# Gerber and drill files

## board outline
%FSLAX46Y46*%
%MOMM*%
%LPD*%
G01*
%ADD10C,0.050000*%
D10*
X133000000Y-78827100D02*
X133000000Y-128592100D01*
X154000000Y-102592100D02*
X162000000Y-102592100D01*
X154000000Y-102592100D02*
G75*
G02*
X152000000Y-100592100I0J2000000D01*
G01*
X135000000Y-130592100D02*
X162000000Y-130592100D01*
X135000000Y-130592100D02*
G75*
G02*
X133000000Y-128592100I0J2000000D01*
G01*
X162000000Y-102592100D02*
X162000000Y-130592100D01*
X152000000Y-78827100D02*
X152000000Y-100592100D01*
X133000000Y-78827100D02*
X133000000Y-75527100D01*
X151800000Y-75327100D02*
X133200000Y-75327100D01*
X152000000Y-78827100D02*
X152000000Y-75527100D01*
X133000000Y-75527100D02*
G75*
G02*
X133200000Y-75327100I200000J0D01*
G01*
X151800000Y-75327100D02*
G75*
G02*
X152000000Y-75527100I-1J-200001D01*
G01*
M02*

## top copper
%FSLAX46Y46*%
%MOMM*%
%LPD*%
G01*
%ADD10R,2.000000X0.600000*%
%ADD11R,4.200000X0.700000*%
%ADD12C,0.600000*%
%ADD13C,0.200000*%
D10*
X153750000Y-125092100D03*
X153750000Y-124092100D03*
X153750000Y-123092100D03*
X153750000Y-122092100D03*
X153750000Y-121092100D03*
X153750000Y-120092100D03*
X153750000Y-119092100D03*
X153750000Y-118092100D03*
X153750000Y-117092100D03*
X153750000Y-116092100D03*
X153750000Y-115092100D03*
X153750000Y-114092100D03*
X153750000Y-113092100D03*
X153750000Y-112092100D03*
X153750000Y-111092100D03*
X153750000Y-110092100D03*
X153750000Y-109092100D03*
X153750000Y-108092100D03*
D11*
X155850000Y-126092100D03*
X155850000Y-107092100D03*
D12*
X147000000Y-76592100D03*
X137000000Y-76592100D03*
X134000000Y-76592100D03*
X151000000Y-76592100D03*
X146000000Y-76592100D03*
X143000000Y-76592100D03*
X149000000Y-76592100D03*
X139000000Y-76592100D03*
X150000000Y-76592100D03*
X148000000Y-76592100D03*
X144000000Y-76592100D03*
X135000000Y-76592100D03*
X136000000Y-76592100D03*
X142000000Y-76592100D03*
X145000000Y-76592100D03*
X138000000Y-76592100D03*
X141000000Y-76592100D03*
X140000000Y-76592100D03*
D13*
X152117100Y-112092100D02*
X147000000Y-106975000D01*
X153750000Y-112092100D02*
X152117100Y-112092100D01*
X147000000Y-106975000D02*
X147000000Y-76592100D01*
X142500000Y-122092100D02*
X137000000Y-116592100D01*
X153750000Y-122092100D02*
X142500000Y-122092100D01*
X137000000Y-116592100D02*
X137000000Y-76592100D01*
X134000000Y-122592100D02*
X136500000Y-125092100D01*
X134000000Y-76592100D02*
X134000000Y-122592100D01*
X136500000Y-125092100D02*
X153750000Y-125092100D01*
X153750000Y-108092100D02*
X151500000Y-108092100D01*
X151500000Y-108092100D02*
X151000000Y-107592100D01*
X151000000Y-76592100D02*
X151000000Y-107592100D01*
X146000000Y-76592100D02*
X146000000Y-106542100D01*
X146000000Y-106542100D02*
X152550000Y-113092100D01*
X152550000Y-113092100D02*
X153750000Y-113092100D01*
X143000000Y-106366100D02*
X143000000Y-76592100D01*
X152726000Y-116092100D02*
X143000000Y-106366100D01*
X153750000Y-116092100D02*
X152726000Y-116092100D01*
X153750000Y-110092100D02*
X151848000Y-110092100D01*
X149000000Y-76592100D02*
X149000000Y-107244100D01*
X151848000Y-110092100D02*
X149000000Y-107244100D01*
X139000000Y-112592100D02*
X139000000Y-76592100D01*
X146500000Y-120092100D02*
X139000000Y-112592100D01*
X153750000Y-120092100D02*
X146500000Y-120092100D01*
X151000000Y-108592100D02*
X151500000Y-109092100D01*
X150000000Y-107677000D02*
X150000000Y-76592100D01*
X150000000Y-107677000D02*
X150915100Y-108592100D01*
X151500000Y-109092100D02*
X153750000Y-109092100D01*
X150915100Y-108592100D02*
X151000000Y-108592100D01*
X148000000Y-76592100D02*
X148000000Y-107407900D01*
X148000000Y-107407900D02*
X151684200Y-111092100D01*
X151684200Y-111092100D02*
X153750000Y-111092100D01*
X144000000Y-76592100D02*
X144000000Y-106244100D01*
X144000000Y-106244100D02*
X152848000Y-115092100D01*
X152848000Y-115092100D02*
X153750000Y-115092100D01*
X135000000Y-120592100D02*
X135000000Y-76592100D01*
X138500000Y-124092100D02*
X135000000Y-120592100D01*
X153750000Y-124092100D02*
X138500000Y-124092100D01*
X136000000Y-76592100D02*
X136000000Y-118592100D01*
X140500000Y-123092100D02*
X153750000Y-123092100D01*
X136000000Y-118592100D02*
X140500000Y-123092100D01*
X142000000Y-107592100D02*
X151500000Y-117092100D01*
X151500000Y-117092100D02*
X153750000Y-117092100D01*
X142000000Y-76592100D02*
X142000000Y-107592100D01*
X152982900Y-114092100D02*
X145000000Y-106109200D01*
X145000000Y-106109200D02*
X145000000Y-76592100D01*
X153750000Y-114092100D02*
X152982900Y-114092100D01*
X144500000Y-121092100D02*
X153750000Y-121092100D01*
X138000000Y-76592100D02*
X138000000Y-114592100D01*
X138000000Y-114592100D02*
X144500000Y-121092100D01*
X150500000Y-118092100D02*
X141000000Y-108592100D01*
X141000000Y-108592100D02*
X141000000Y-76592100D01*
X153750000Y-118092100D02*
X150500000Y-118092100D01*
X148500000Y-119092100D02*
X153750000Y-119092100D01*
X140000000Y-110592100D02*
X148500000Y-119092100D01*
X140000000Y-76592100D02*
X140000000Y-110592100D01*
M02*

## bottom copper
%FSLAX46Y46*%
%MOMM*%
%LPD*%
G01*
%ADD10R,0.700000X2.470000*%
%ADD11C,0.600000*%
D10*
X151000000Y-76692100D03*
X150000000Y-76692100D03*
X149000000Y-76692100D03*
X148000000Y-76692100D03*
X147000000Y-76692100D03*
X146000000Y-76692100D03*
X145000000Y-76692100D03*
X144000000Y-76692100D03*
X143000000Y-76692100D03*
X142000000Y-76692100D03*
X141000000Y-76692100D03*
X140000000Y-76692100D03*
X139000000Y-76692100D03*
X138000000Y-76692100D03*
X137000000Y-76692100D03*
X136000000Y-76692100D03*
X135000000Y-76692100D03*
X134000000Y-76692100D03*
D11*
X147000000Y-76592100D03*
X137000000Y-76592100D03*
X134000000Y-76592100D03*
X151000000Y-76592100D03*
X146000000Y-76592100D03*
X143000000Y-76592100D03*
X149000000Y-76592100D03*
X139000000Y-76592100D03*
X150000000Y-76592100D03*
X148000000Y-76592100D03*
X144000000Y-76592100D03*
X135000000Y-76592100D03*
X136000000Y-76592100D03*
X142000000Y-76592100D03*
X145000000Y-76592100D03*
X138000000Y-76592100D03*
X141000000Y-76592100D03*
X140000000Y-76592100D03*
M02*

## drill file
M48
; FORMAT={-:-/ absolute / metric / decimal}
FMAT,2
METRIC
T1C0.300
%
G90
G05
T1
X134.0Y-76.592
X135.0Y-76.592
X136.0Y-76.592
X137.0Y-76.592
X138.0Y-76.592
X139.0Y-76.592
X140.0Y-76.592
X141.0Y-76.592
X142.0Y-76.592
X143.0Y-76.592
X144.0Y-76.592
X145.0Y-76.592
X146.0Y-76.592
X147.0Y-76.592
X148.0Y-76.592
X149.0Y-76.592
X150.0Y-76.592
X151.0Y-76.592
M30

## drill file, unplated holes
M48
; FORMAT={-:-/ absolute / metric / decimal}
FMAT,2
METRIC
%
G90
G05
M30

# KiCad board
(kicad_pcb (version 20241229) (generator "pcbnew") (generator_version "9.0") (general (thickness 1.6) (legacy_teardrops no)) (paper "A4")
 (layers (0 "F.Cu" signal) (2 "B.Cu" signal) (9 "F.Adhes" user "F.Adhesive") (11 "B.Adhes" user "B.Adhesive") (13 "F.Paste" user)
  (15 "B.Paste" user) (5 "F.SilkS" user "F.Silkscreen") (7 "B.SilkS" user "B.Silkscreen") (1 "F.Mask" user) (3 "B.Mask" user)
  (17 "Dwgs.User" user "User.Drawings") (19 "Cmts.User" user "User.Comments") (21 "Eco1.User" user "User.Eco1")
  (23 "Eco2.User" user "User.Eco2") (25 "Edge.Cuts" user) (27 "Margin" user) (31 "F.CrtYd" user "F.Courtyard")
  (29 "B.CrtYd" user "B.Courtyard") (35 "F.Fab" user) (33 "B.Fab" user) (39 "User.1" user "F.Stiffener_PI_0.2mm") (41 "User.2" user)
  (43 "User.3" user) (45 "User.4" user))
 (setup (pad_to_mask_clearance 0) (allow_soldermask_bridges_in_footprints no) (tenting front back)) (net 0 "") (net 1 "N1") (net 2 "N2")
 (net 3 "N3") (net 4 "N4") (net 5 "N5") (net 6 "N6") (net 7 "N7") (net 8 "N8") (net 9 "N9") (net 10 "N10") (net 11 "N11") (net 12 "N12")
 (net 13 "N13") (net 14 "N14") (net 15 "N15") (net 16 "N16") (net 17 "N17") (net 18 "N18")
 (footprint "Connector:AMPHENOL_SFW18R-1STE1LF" (layer "F.Cu") (at 157 116.5921 90)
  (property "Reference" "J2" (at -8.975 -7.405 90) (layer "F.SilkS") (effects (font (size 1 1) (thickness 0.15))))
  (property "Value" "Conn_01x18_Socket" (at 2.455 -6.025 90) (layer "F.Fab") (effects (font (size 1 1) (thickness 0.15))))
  (pad "1" smd rect (at -8.5 -3.25 90) (size 0.6 2) (layers "F.Cu" "F.Mask" "F.Paste") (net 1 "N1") (solder_mask_margin 0.102))
  (pad "2" smd rect (at -7.5 -3.25 90) (size 0.6 2) (layers "F.Cu" "F.Mask" "F.Paste") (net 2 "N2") (solder_mask_margin 0.102))
  (pad "3" smd rect (at -6.5 -3.25 90) (size 0.6 2) (layers "F.Cu" "F.Mask" "F.Paste") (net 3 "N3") (solder_mask_margin 0.102))
  (pad "4" smd rect (at -5.5 -3.25 90) (size 0.6 2) (layers "F.Cu" "F.Mask" "F.Paste") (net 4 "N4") (solder_mask_margin 0.102))
  (pad "5" smd rect (at -4.5 -3.25 90) (size 0.6 2) (layers "F.Cu" "F.Mask" "F.Paste") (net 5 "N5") (solder_mask_margin 0.102))
  (pad "6" smd rect (at -3.5 -3.25 90) (size 0.6 2) (layers "F.Cu" "F.Mask" "F.Paste") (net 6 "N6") (solder_mask_margin 0.102))
  (pad "7" smd rect (at -2.5 -3.25 90) (size 0.6 2) (layers "F.Cu" "F.Mask" "F.Paste") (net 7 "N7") (solder_mask_margin 0.102))
  (pad "8" smd rect (at -1.5 -3.25 90) (size 0.6 2) (layers "F.Cu" "F.Mask" "F.Paste") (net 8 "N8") (solder_mask_margin 0.102))
  (pad "9" smd rect (at -0.5 -3.25 90) (size 0.6 2) (layers "F.Cu" "F.Mask" "F.Paste") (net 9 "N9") (solder_mask_margin 0.102))
  (pad "10" smd rect (at 0.5 -3.25 90) (size 0.6 2) (layers "F.Cu" "F.Mask" "F.Paste") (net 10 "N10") (solder_mask_margin 0.102))
  (pad "11" smd rect (at 1.5 -3.25 90) (size 0.6 2) (layers "F.Cu" "F.Mask" "F.Paste") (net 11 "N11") (solder_mask_margin 0.102))
  (pad "12" smd rect (at 2.5 -3.25 90) (size 0.6 2) (layers "F.Cu" "F.Mask" "F.Paste") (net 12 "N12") (solder_mask_margin 0.102))
  (pad "13" smd rect (at 3.5 -3.25 90) (size 0.6 2) (layers "F.Cu" "F.Mask" "F.Paste") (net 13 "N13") (solder_mask_margin 0.102))
  (pad "14" smd rect (at 4.5 -3.25 90) (size 0.6 2) (layers "F.Cu" "F.Mask" "F.Paste") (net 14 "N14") (solder_mask_margin 0.102))
  (pad "15" smd rect (at 5.5 -3.25 90) (size 0.6 2) (layers "F.Cu" "F.Mask" "F.Paste") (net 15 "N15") (solder_mask_margin 0.102))
  (pad "16" smd rect (at 6.5 -3.25 90) (size 0.6 2) (layers "F.Cu" "F.Mask" "F.Paste") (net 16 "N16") (solder_mask_margin 0.102))
  (pad "17" smd rect (at 7.5 -3.25 90) (size 0.6 2) (layers "F.Cu" "F.Mask" "F.Paste") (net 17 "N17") (solder_mask_margin 0.102))
  (pad "18" smd rect (at 8.5 -3.25 90) (size 0.6 2) (layers "F.Cu" "F.Mask" "F.Paste") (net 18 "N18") (solder_mask_margin 0.102))
  (pad "S1" smd rect (at -9.5 -1.15 90) (size 0.7 4.2) (layers "F.Cu" "F.Mask" "F.Paste") (solder_mask_margin 0.102))
  (pad "S2" smd rect (at 9.5 -1.15 90) (size 0.7 4.2) (layers "F.Cu" "F.Mask" "F.Paste") (solder_mask_margin 0.102)))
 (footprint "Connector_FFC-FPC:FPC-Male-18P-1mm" (layer "B.Cu") (at 142.91 76.6321 180)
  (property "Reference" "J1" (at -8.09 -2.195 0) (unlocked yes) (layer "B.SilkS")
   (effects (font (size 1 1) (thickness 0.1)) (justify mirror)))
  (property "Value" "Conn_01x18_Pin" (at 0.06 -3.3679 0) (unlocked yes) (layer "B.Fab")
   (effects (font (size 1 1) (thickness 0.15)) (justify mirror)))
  (fp_line (start 9.91 -2.195) (end 9.91 1.105) (stroke (width 0.05) (type default)) (layer "Edge.Cuts"))
  (fp_line (start -8.89 1.305) (end 9.71 1.305) (stroke (width 0.05) (type default)) (layer "Edge.Cuts"))
  (fp_line (start -9.09 -2.195) (end -9.09 1.105) (stroke (width 0.05) (type default)) (layer "Edge.Cuts"))
  (fp_arc (start 9.91 1.105) (mid 9.851421 1.246421) (end 9.71 1.305) (stroke (width 0.05) (type default)) (layer "Edge.Cuts"))
  (fp_arc (start -8.89 1.305) (mid -9.031421 1.246421) (end -9.09 1.105) (stroke (width 0.05) (type default)) (layer "Edge.Cuts"))
  (pad "1" smd rect (at -8.09 -0.06 90) (size 2.47 0.7) (layers "B.Cu" "B.Mask" "B.Paste") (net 18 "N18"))
  (pad "2" smd rect (at -7.09 -0.06 90) (size 2.47 0.7) (layers "B.Cu" "B.Mask" "B.Paste") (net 17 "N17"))
  (pad "3" smd rect (at -6.09 -0.06 90) (size 2.47 0.7) (layers "B.Cu" "B.Mask" "B.Paste") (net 16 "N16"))
  (pad "4" smd rect (at -5.09 -0.06 90) (size 2.47 0.7) (layers "B.Cu" "B.Mask" "B.Paste") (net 15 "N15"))
  (pad "5" smd rect (at -4.09 -0.06 90) (size 2.47 0.7) (layers "B.Cu" "B.Mask" "B.Paste") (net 14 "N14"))
  (pad "6" smd rect (at -3.09 -0.06 90) (size 2.47 0.7) (layers "B.Cu" "B.Mask" "B.Paste") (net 13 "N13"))
  (pad "7" smd rect (at -2.09 -0.06 90) (size 2.47 0.7) (layers "B.Cu" "B.Mask" "B.Paste") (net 12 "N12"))
  (pad "8" smd rect (at -1.09 -0.06 90) (size 2.47 0.7) (layers "B.Cu" "B.Mask" "B.Paste") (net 11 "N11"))
  (pad "9" smd rect (at -0.09 -0.06 90) (size 2.47 0.7) (layers "B.Cu" "B.Mask" "B.Paste") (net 10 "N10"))
  (pad "10" smd rect (at 0.91 -0.06 90) (size 2.47 0.7) (layers "B.Cu" "B.Mask" "B.Paste") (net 9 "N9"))
  (pad "11" smd rect (at 1.91 -0.06 90) (size 2.47 0.7) (layers "B.Cu" "B.Mask" "B.Paste") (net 8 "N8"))
  (pad "12" smd rect (at 2.91 -0.06 90) (size 2.47 0.7) (layers "B.Cu" "B.Mask" "B.Paste") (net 7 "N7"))
  (pad "13" smd rect (at 3.91 -0.06 90) (size 2.47 0.7) (layers "B.Cu" "B.Mask" "B.Paste") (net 6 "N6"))
  (pad "14" smd rect (at 4.91 -0.06 90) (size 2.47 0.7) (layers "B.Cu" "B.Mask" "B.Paste") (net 5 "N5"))
  (pad "15" smd rect (at 5.91 -0.06 90) (size 2.47 0.7) (layers "B.Cu" "B.Mask" "B.Paste") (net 4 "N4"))
  (pad "16" smd rect (at 6.91 -0.06 90) (size 2.47 0.7) (layers "B.Cu" "B.Mask" "B.Paste") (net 3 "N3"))
  (pad "17" smd rect (at 7.91 -0.06 90) (size 2.47 0.7) (layers "B.Cu" "B.Mask" "B.Paste") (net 2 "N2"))
  (pad "18" smd rect (at 8.91 -0.06 90) (size 2.47 0.7) (layers "B.Cu" "B.Mask" "B.Paste") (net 1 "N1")))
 (gr_line (start 133 78.8271) (end 133 128.5921) (stroke (width 0.05) (type default)) (layer "Edge.Cuts"))
 (gr_line (start 154 102.5921) (end 162 102.5921) (stroke (width 0.05) (type default)) (layer "Edge.Cuts"))
 (gr_arc (start 154 102.5921) (mid 152.585786 102.006314) (end 152 100.5921) (stroke (width 0.05) (type default)) (layer "Edge.Cuts"))
 (gr_line (start 135 130.5921) (end 162 130.5921) (stroke (width 0.05) (type default)) (layer "Edge.Cuts"))
 (gr_arc (start 135 130.5921) (mid 133.585786 130.006314) (end 133 128.5921) (stroke (width 0.05) (type default)) (layer "Edge.Cuts"))
 (gr_line (start 162 102.5921) (end 162 130.5921) (stroke (width 0.05) (type default)) (layer "Edge.Cuts"))
 (gr_line (start 152 78.8271) (end 152 100.5921) (stroke (width 0.05) (type default)) (layer "Edge.Cuts"))
 (segment (start 152.1171 112.0921) (end 147 106.975) (width 0.2) (layer "F.Cu") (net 14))
 (segment (start 153.75 112.0921) (end 152.1171 112.0921) (width 0.2) (layer "F.Cu") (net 14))
 (segment (start 147 106.975) (end 147 76.5921) (width 0.2) (layer "F.Cu") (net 14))
 (via (at 147 76.5921) (size 0.6) (drill 0.3) (layers "F.Cu" "B.Cu") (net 14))
 (segment (start 142.5 122.0921) (end 137 116.5921) (width 0.2) (layer "F.Cu") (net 4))
 (segment (start 153.75 122.0921) (end 142.5 122.0921) (width 0.2) (layer "F.Cu") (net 4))
 (segment (start 137 116.5921) (end 137 76.5921) (width 0.2) (layer "F.Cu") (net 4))
 (via (at 137 76.5921) (size 0.6) (drill 0.3) (layers "F.Cu" "B.Cu") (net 4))
 (segment (start 134 122.5921) (end 136.5 125.0921) (width 0.2) (layer "F.Cu") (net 1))
 (segment (start 134 76.5921) (end 134 122.5921) (width 0.2) (layer "F.Cu") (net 1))
 (segment (start 136.5 125.0921) (end 153.75 125.0921) (width 0.2) (layer "F.Cu") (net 1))
 (via (at 134 76.5921) (size 0.6) (drill 0.3) (layers "F.Cu" "B.Cu") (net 1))
 (segment (start 153.75 108.0921) (end 151.5 108.0921) (width 0.2) (layer "F.Cu") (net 18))
 (segment (start 151.5 108.0921) (end 151 107.5921) (width 0.2) (layer "F.Cu") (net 18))
 (segment (start 151 76.5921) (end 151 107.5921) (width 0.2) (layer "F.Cu") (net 18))
 (via (at 151 76.5921) (size 0.6) (drill 0.3) (layers "F.Cu" "B.Cu") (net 18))
 (segment (start 146 76.5921) (end 146 106.5421) (width 0.2) (layer "F.Cu") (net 13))
 (segment (start 146 106.5421) (end 152.55 113.0921) (width 0.2) (layer "F.Cu") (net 13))
 (segment (start 152.55 113.0921) (end 153.75 113.0921) (width 0.2) (layer "F.Cu") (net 13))
 (via (at 146 76.5921) (size 0.6) (drill 0.3) (layers "F.Cu" "B.Cu") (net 13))
 (segment (start 143 106.3661) (end 143 76.5921) (width 0.2) (layer "F.Cu") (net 10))
 (segment (start 152.726 116.0921) (end 143 106.3661) (width 0.2) (layer "F.Cu") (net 10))
 (segment (start 153.75 116.0921) (end 152.726 116.0921) (width 0.2) (layer "F.Cu") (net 10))
 (via (at 143 76.5921) (size 0.6) (drill 0.3) (layers "F.Cu" "B.Cu") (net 10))
 (segment (start 153.75 110.0921) (end 151.848 110.0921) (width 0.2) (layer "F.Cu") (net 16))
 (segment (start 149 76.5921) (end 149 107.2441) (width 0.2) (layer "F.Cu") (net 16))
 (segment (start 151.848 110.0921) (end 149 107.2441) (width 0.2) (layer "F.Cu") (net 16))
 (via (at 149 76.5921) (size 0.6) (drill 0.3) (layers "F.Cu" "B.Cu") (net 16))
 (segment (start 139 112.5921) (end 139 76.5921) (width 0.2) (layer "F.Cu") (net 6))
 (segment (start 146.5 120.0921) (end 139 112.5921) (width 0.2) (layer "F.Cu") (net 6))
 (segment (start 153.75 120.0921) (end 146.5 120.0921) (width 0.2) (layer "F.Cu") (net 6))
 (via (at 139 76.5921) (size 0.6) (drill 0.3) (layers "F.Cu" "B.Cu") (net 6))
 (segment (start 151 108.5921) (end 151.5 109.0921) (width 0.2) (layer "F.Cu") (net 17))
 (segment (start 150 107.677) (end 150 76.5921) (width 0.2) (layer "F.Cu") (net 17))
 (segment (start 150 107.677) (end 150.9151 108.5921) (width 0.2) (layer "F.Cu") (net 17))
 (segment (start 151.5 109.0921) (end 153.75 109.0921) (width 0.2) (layer "F.Cu") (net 17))
 (segment (start 150.9151 108.5921) (end 151 108.5921) (width 0.2) (layer "F.Cu") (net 17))
 (via (at 150 76.5921) (size 0.6) (drill 0.3) (layers "F.Cu" "B.Cu") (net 17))
 (segment (start 148 76.5921) (end 148 107.4079) (width 0.2) (layer "F.Cu") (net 15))
 (segment (start 148 107.4079) (end 151.6842 111.0921) (width 0.2) (layer "F.Cu") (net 15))
 (segment (start 151.6842 111.0921) (end 153.75 111.0921) (width 0.2) (layer "F.Cu") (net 15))
 (via (at 148 76.5921) (size 0.6) (drill 0.3) (layers "F.Cu" "B.Cu") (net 15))
 (segment (start 144 76.5921) (end 144 106.2441) (width 0.2) (layer "F.Cu") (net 11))
 (segment (start 144 106.2441) (end 152.848 115.0921) (width 0.2) (layer "F.Cu") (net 11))
 (segment (start 152.848 115.0921) (end 153.75 115.0921) (width 0.2) (layer "F.Cu") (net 11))
 (via (at 144 76.5921) (size 0.6) (drill 0.3) (layers "F.Cu" "B.Cu") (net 11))
 (segment (start 135 120.5921) (end 135 76.5921) (width 0.2) (layer "F.Cu") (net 2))
 (segment (start 138.5 124.0921) (end 135 120.5921) (width 0.2) (layer "F.Cu") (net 2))
 (segment (start 153.75 124.0921) (end 138.5 124.0921) (width 0.2) (layer "F.Cu") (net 2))
 (via (at 135 76.5921) (size 0.6) (drill 0.3) (layers "F.Cu" "B.Cu") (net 2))
 (segment (start 136 76.5921) (end 136 118.5921) (width 0.2) (layer "F.Cu") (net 3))
 (segment (start 140.5 123.0921) (end 153.75 123.0921) (width 0.2) (layer "F.Cu") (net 3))
 (segment (start 136 118.5921) (end 140.5 123.0921) (width 0.2) (layer "F.Cu") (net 3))
 (via (at 136 76.5921) (size 0.6) (drill 0.3) (layers "F.Cu" "B.Cu") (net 3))
 (segment (start 142 107.5921) (end 151.5 117.0921) (width 0.2) (layer "F.Cu") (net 9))
 (segment (start 151.5 117.0921) (end 153.75 117.0921) (width 0.2) (layer "F.Cu") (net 9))
 (segment (start 142 76.5921) (end 142 107.5921) (width 0.2) (layer "F.Cu") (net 9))
 (via (at 142 76.5921) (size 0.6) (drill 0.3) (layers "F.Cu" "B.Cu") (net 9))
 (segment (start 152.9829 114.0921) (end 145 106.1092) (width 0.2) (layer "F.Cu") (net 12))
 (segment (start 145 106.1092) (end 145 76.5921) (width 0.2) (layer "F.Cu") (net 12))
 (segment (start 153.75 114.0921) (end 152.9829 114.0921) (width 0.2) (layer "F.Cu") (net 12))
 (via (at 145 76.5921) (size 0.6) (drill 0.3) (layers "F.Cu" "B.Cu") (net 12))
 (segment (start 144.5 121.0921) (end 153.75 121.0921) (width 0.2) (layer "F.Cu") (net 5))
 (segment (start 138 76.5921) (end 138 114.5921) (width 0.2) (layer "F.Cu") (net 5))
 (segment (start 138 114.5921) (end 144.5 121.0921) (width 0.2) (layer "F.Cu") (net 5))
 (via (at 138 76.5921) (size 0.6) (drill 0.3) (layers "F.Cu" "B.Cu") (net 5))
 (segment (start 150.5 118.0921) (end 141 108.5921) (width 0.2) (layer "F.Cu") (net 8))
 (segment (start 141 108.5921) (end 141 76.5921) (width 0.2) (layer "F.Cu") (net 8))
 (segment (start 153.75 118.0921) (end 150.5 118.0921) (width 0.2) (layer "F.Cu") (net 8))
 (via (at 141 76.5921) (size 0.6) (drill 0.3) (layers "F.Cu" "B.Cu") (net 8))
 (segment (start 148.5 119.0921) (end 153.75 119.0921) (width 0.2) (layer "F.Cu") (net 7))
 (segment (start 140 110.5921) (end 148.5 119.0921) (width 0.2) (layer "F.Cu") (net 7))
 (segment (start 140 76.5921) (end 140 110.5921) (width 0.2) (layer "F.Cu") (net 7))
 (via (at 140 76.5921) (size 0.6) (drill 0.3) (layers "F.Cu" "B.Cu") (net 7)))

